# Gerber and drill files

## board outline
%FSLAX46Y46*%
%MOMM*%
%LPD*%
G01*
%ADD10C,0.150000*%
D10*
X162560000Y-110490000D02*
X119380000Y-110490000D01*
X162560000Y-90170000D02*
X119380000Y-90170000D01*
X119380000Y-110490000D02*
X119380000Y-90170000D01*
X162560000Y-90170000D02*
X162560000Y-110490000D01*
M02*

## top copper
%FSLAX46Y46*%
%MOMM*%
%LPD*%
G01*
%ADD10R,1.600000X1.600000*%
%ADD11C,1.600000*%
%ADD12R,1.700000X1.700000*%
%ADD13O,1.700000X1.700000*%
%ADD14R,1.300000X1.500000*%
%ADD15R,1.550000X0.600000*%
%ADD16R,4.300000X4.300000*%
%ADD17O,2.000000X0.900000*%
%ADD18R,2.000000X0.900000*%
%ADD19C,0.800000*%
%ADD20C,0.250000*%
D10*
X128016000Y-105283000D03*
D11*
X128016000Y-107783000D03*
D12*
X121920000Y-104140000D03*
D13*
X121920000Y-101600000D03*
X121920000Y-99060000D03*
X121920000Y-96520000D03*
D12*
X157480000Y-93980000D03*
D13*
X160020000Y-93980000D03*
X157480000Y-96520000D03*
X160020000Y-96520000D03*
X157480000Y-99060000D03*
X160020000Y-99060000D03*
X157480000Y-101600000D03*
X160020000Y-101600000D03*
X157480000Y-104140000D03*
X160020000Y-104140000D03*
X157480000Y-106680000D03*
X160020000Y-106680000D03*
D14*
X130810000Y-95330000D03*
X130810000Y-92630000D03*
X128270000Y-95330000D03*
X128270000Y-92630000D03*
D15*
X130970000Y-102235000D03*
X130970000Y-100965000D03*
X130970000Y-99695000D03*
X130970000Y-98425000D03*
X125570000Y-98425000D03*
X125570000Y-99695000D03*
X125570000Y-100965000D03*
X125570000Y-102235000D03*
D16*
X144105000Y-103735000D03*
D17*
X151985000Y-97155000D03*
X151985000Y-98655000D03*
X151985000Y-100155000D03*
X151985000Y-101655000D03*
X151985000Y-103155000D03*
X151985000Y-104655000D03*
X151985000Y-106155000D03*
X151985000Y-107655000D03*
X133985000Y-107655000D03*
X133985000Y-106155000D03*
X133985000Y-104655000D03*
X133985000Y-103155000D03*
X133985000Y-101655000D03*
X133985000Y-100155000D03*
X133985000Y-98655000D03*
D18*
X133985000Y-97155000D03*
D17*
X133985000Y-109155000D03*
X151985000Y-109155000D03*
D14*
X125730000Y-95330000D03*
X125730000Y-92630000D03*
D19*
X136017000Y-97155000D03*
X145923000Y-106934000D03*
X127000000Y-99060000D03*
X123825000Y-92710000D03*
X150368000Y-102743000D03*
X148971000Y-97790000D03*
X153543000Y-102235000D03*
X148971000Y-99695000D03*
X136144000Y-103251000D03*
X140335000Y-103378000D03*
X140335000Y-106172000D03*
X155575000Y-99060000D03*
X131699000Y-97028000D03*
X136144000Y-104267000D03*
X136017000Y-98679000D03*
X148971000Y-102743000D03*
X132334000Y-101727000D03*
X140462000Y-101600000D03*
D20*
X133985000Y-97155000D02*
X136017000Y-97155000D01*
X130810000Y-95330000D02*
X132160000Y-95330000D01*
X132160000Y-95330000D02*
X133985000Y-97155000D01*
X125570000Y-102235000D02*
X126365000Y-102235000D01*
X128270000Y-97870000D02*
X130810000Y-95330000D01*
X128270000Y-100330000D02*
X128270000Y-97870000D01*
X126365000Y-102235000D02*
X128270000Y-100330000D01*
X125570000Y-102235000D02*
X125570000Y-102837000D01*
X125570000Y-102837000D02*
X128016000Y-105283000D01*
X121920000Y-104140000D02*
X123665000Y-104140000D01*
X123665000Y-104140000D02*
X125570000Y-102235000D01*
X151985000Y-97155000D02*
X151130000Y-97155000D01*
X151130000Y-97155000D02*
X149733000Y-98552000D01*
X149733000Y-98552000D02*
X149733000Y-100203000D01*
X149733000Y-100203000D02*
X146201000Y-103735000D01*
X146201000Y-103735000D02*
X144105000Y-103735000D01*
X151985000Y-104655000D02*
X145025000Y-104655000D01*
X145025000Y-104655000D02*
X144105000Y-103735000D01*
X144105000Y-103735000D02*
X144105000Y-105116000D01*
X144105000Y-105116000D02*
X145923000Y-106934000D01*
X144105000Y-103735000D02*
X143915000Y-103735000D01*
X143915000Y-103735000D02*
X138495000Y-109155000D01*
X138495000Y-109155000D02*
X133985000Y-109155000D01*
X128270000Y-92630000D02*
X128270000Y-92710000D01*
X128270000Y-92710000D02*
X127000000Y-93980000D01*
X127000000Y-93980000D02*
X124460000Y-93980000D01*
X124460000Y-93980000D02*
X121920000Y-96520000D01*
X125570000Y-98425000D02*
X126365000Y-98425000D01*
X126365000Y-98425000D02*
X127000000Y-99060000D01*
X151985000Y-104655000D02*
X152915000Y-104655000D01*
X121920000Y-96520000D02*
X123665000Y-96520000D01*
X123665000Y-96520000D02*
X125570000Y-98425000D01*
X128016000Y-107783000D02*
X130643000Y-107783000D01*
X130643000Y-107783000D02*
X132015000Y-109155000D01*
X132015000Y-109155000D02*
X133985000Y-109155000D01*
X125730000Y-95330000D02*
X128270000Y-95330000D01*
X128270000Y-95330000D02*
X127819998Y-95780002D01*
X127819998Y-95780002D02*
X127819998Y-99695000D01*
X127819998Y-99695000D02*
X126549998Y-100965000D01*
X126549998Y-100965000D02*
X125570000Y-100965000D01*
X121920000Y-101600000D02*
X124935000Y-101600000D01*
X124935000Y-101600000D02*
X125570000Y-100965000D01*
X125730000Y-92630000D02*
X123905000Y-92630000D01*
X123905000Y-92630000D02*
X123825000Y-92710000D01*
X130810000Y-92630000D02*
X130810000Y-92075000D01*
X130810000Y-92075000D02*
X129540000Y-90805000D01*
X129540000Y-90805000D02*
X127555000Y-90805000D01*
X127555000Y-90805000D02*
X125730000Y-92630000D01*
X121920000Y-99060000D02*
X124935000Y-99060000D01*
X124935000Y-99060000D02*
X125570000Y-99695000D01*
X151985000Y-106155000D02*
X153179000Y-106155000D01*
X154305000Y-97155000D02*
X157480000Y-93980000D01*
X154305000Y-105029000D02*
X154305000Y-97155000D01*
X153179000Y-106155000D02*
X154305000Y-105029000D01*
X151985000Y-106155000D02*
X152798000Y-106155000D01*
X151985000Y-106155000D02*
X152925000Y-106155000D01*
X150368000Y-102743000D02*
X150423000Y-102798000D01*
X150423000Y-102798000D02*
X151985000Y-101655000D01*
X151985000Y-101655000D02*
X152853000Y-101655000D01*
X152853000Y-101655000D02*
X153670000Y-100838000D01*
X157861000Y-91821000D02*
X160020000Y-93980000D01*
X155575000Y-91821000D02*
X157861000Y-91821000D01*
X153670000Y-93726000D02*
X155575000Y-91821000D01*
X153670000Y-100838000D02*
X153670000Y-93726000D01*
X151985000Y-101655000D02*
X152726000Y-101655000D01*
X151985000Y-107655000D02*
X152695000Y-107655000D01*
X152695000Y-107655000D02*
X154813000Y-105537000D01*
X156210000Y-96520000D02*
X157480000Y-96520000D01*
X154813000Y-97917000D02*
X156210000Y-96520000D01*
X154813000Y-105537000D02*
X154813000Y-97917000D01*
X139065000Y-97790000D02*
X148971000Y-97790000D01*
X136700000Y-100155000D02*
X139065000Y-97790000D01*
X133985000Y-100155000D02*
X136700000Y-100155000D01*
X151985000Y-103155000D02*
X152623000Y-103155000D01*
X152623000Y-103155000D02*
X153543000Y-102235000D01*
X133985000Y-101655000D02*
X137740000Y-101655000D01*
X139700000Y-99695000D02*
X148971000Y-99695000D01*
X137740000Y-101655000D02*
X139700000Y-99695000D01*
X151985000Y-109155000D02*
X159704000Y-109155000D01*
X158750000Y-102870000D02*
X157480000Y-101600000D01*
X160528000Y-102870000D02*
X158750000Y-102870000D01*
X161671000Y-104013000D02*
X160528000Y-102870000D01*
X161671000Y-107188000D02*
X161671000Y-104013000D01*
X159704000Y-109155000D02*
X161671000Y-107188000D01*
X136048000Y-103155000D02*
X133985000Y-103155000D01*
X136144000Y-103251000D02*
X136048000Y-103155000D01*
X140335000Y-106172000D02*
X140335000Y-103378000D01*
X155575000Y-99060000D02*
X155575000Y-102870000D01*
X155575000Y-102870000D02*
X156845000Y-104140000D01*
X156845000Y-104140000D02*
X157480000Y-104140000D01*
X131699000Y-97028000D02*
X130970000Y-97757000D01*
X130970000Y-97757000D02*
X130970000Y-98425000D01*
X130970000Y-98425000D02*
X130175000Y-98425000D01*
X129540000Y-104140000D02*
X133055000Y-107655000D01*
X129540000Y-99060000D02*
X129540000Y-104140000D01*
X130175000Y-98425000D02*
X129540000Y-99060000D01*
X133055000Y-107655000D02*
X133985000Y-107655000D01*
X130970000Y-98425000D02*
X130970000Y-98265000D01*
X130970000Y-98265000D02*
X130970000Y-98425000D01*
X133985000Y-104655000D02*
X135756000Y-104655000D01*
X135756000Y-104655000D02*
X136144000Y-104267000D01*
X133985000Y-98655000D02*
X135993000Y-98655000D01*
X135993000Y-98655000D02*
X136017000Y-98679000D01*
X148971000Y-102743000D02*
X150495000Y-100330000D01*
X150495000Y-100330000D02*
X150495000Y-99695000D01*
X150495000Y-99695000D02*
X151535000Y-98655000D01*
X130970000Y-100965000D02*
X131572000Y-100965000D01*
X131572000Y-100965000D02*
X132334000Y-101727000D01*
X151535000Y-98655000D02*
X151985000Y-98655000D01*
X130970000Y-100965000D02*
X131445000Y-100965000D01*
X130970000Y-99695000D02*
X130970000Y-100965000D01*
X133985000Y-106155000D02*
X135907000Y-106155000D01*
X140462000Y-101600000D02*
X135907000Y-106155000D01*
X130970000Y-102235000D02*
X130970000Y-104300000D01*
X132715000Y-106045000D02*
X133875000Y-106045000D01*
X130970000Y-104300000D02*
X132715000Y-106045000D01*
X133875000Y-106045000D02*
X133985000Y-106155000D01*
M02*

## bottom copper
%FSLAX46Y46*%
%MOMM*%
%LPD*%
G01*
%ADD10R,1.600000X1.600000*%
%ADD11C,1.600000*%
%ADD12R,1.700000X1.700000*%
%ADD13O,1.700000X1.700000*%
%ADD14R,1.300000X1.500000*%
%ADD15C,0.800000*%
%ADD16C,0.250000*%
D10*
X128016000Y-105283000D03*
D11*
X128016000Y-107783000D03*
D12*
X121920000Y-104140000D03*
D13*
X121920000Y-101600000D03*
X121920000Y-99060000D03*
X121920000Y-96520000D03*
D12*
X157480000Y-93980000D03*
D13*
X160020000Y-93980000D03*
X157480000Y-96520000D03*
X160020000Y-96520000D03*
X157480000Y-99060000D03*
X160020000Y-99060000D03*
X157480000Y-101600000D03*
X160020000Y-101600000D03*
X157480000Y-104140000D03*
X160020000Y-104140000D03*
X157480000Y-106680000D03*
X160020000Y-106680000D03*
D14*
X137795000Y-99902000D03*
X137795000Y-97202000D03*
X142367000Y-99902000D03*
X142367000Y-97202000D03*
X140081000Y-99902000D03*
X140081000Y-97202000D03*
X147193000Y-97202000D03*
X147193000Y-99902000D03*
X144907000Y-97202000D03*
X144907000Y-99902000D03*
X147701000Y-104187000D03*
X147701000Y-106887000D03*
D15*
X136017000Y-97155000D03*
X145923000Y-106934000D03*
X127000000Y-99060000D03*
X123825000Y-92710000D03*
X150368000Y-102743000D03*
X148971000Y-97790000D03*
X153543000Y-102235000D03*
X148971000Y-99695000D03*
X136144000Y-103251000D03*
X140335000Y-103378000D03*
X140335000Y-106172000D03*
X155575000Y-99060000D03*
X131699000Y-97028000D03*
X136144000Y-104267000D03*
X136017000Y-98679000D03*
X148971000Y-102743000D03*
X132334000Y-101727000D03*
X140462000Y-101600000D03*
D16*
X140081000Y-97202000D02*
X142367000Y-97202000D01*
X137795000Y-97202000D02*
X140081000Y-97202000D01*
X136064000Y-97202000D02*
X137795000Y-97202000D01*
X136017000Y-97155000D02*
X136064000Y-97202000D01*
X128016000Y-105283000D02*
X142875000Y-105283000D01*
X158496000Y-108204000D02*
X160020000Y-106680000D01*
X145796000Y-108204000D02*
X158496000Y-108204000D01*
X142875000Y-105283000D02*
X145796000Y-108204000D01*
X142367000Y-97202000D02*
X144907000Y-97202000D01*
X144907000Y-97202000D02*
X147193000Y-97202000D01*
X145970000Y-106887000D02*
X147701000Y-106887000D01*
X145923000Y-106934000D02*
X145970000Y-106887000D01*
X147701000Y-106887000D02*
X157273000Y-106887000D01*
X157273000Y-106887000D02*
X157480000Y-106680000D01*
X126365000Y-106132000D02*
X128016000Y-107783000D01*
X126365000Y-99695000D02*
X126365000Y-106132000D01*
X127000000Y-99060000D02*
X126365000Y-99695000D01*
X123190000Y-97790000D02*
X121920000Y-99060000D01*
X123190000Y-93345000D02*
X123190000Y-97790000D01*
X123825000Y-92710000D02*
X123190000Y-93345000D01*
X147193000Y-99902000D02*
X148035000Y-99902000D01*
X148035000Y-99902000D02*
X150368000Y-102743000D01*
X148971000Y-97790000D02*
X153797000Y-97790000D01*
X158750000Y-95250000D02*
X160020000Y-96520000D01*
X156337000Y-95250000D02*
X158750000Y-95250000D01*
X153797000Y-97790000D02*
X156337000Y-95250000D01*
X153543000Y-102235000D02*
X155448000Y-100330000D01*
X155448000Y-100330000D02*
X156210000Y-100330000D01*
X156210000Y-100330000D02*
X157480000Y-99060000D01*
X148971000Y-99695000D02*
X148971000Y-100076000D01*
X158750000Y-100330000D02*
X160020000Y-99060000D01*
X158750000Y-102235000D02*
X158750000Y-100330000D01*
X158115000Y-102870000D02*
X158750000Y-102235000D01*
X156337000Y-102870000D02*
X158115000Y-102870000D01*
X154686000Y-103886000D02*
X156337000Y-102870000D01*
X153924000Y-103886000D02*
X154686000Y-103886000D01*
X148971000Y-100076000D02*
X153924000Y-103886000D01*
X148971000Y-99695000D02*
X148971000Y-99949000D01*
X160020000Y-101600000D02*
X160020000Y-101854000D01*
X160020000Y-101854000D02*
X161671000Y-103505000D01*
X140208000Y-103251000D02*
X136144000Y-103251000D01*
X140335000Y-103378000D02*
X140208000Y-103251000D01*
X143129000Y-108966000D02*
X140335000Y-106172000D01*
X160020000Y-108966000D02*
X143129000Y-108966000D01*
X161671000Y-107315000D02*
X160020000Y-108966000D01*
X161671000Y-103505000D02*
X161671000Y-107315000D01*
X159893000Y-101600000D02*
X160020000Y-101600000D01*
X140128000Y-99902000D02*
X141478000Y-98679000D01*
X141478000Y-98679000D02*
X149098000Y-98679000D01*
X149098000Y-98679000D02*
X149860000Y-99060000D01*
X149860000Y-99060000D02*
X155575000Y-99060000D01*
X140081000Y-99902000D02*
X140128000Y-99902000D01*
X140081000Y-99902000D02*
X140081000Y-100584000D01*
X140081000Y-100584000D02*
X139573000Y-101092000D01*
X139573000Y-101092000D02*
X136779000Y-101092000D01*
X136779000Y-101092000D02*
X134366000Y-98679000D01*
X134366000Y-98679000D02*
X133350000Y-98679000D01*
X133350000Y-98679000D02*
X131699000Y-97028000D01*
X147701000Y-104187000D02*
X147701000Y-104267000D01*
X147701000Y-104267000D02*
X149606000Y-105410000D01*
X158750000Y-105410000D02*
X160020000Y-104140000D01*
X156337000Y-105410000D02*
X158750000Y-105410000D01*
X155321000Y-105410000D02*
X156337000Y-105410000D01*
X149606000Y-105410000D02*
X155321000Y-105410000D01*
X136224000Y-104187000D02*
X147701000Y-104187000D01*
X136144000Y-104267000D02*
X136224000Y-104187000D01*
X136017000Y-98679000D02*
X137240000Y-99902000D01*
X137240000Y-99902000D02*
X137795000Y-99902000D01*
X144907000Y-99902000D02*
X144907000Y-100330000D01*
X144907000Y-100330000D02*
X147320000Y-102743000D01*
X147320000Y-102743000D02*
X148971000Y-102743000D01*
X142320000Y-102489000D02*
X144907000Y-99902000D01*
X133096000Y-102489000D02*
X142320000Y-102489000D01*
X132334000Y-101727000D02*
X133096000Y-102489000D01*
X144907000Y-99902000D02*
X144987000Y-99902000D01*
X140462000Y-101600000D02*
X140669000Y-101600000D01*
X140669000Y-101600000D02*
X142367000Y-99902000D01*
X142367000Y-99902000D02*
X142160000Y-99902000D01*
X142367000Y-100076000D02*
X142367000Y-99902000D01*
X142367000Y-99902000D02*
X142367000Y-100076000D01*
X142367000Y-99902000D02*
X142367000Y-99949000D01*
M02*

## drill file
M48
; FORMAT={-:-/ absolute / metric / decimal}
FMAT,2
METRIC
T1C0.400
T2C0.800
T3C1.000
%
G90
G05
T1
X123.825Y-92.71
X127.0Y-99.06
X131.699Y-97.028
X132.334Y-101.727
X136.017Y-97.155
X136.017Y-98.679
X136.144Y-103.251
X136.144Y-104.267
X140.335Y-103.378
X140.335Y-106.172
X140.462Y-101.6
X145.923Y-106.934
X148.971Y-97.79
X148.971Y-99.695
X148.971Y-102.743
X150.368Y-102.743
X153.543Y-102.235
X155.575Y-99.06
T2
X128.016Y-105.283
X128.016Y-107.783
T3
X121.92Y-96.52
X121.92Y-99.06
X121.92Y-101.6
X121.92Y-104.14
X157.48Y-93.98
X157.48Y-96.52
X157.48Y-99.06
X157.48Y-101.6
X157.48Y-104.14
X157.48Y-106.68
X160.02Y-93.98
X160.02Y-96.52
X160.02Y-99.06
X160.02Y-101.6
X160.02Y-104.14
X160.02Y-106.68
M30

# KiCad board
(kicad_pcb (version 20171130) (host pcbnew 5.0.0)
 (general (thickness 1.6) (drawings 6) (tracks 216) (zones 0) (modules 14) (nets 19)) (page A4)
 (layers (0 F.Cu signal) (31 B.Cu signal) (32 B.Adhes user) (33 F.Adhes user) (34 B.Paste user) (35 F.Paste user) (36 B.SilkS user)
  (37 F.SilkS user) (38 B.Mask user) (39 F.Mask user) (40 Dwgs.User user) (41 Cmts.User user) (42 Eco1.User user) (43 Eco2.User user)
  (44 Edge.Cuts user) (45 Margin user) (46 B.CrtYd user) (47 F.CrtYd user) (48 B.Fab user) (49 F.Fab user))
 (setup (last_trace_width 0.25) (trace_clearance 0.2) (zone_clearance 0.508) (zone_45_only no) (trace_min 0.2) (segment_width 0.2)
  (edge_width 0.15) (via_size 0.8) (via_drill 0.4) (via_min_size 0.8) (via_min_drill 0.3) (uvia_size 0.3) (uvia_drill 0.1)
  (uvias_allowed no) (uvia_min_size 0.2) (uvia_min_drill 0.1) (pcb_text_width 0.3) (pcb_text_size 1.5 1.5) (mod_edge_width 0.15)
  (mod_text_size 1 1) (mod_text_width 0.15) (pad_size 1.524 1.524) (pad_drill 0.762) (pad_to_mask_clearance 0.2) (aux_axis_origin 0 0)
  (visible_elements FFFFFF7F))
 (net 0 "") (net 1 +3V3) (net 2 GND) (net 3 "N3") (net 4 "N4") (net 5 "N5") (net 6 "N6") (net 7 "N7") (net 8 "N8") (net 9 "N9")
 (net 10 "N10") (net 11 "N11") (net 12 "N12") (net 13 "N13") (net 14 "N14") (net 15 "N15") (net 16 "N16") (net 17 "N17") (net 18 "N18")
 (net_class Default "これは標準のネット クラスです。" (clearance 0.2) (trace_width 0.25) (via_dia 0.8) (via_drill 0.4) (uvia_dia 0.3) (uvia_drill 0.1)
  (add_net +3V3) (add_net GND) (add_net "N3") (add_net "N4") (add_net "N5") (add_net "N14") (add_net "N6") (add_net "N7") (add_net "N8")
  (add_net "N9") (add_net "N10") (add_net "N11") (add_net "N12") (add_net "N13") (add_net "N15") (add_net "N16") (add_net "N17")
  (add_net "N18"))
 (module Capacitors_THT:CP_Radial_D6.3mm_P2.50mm (layer F.Cu) (at 128.016 105.283 270)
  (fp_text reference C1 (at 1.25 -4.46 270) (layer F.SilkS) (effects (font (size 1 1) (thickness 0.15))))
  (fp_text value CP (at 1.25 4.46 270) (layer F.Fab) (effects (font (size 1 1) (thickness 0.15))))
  (pad 1 thru_hole rect (at 0 0 270) (size 1.6 1.6) (drill 0.8) (layers *.Cu *.Mask) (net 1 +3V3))
  (pad 2 thru_hole circle (at 2.5 0 270) (size 1.6 1.6) (drill 0.8) (layers *.Cu *.Mask) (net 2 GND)))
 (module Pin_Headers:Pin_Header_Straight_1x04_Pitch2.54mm (layer F.Cu) (at 121.92 104.14 180)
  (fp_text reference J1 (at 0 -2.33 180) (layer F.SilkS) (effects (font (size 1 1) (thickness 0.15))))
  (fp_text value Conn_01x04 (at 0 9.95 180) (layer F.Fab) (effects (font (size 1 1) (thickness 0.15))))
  (pad 1 thru_hole rect (at 0 0 180) (size 1.7 1.7) (drill 1) (layers *.Cu *.Mask) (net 1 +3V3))
  (pad 2 thru_hole oval (at 0 2.54 180) (size 1.7 1.7) (drill 1) (layers *.Cu *.Mask) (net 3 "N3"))
  (pad 3 thru_hole oval (at 0 5.08 180) (size 1.7 1.7) (drill 1) (layers *.Cu *.Mask) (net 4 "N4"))
  (pad 4 thru_hole oval (at 0 7.62 180) (size 1.7 1.7) (drill 1) (layers *.Cu *.Mask) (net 2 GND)))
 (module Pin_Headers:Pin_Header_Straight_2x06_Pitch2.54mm (layer F.Cu) (at 157.48 93.98)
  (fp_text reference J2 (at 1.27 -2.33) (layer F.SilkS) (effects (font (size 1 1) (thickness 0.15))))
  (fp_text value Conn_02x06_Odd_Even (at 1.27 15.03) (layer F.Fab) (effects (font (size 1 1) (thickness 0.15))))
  (pad 1 thru_hole rect (at 0 0) (size 1.7 1.7) (drill 1) (layers *.Cu *.Mask) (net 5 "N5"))
  (pad 2 thru_hole oval (at 2.54 0) (size 1.7 1.7) (drill 1) (layers *.Cu *.Mask) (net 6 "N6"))
  (pad 3 thru_hole oval (at 0 2.54) (size 1.7 1.7) (drill 1) (layers *.Cu *.Mask) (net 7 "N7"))
  (pad 4 thru_hole oval (at 2.54 2.54) (size 1.7 1.7) (drill 1) (layers *.Cu *.Mask) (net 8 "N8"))
  (pad 5 thru_hole oval (at 0 5.08) (size 1.7 1.7) (drill 1) (layers *.Cu *.Mask) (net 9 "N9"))
  (pad 6 thru_hole oval (at 2.54 5.08) (size 1.7 1.7) (drill 1) (layers *.Cu *.Mask) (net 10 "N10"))
  (pad 7 thru_hole oval (at 0 7.62) (size 1.7 1.7) (drill 1) (layers *.Cu *.Mask) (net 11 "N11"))
  (pad 8 thru_hole oval (at 2.54 7.62) (size 1.7 1.7) (drill 1) (layers *.Cu *.Mask) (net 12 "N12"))
  (pad 9 thru_hole oval (at 0 10.16) (size 1.7 1.7) (drill 1) (layers *.Cu *.Mask) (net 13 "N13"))
  (pad 10 thru_hole oval (at 2.54 10.16) (size 1.7 1.7) (drill 1) (layers *.Cu *.Mask) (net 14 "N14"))
  (pad 11 thru_hole oval (at 0 12.7) (size 1.7 1.7) (drill 1) (layers *.Cu *.Mask) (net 2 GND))
  (pad 12 thru_hole oval (at 2.54 12.7) (size 1.7 1.7) (drill 1) (layers *.Cu *.Mask) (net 1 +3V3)))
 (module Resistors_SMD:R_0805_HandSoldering (layer B.Cu) (at 137.795 98.552 90)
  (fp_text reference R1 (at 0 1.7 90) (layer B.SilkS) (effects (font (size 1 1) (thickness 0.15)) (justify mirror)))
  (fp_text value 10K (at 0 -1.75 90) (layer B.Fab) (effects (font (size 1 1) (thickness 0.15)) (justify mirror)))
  (pad 1 smd rect (at -1.35 0 90) (size 1.5 1.3) (layers B.Cu B.Paste B.Mask) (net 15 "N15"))
  (pad 2 smd rect (at 1.35 0 90) (size 1.5 1.3) (layers B.Cu B.Paste B.Mask) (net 1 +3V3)))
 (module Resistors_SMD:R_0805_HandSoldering (layer B.Cu) (at 142.367 98.552 90)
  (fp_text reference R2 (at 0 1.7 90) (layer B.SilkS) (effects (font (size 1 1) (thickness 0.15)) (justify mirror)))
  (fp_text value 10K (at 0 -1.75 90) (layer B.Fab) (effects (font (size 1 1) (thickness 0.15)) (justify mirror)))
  (pad 1 smd rect (at -1.35 0 90) (size 1.5 1.3) (layers B.Cu B.Paste B.Mask) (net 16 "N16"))
  (pad 2 smd rect (at 1.35 0 90) (size 1.5 1.3) (layers B.Cu B.Paste B.Mask) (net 1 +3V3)))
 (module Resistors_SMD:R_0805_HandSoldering (layer B.Cu) (at 140.081 98.552 90)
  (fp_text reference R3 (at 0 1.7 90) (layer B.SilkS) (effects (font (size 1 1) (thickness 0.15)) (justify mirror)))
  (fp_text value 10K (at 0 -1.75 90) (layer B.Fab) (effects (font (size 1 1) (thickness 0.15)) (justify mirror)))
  (pad 1 smd rect (at -1.35 0 90) (size 1.5 1.3) (layers B.Cu B.Paste B.Mask) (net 13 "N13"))
  (pad 2 smd rect (at 1.35 0 90) (size 1.5 1.3) (layers B.Cu B.Paste B.Mask) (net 1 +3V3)))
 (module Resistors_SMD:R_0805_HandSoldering (layer F.Cu) (at 130.81 93.98 90)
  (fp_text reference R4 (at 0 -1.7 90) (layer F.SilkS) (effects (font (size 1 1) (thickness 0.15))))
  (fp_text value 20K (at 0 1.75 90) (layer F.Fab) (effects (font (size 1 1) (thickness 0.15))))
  (pad 1 smd rect (at -1.35 0 90) (size 1.5 1.3) (layers F.Cu F.Paste F.Mask) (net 1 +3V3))
  (pad 2 smd rect (at 1.35 0 90) (size 1.5 1.3) (layers F.Cu F.Paste F.Mask) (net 4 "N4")))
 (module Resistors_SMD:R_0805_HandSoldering (layer F.Cu) (at 128.27 93.98 90)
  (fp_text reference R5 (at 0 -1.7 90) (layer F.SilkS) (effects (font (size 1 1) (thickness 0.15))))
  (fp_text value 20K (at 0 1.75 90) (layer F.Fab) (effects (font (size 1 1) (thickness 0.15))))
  (pad 1 smd rect (at -1.35 0 90) (size 1.5 1.3) (layers F.Cu F.Paste F.Mask) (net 3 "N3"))
  (pad 2 smd rect (at 1.35 0 90) (size 1.5 1.3) (layers F.Cu F.Paste F.Mask) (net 2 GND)))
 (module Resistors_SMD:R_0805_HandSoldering (layer B.Cu) (at 147.193 98.552 270)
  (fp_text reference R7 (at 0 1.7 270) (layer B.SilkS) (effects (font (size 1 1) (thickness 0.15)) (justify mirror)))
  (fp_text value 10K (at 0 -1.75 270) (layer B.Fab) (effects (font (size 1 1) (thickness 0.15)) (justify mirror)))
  (pad 1 smd rect (at -1.35 0 270) (size 1.5 1.3) (layers B.Cu B.Paste B.Mask) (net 1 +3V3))
  (pad 2 smd rect (at 1.35 0 270) (size 1.5 1.3) (layers B.Cu B.Paste B.Mask) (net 6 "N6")))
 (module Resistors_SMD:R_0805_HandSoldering (layer B.Cu) (at 144.907 98.552 270)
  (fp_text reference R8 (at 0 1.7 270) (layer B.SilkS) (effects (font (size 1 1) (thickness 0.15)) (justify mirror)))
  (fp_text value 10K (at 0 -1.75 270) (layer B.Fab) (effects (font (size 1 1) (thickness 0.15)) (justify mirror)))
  (pad 1 smd rect (at -1.35 0 270) (size 1.5 1.3) (layers B.Cu B.Paste B.Mask) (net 1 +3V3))
  (pad 2 smd rect (at 1.35 0 270) (size 1.5 1.3) (layers B.Cu B.Paste B.Mask) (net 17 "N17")))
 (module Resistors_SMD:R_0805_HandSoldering (layer B.Cu) (at 147.701 105.537 270)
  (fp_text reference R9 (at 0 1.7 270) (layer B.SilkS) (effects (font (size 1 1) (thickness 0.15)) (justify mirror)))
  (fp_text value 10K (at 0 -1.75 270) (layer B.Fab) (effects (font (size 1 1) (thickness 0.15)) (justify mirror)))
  (pad 1 smd rect (at -1.35 0 270) (size 1.5 1.3) (layers B.Cu B.Paste B.Mask) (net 14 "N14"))
  (pad 2 smd rect (at 1.35 0 270) (size 1.5 1.3) (layers B.Cu B.Paste B.Mask) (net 2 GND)))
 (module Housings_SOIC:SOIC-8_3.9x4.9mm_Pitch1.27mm (layer F.Cu) (at 128.27 100.33 180)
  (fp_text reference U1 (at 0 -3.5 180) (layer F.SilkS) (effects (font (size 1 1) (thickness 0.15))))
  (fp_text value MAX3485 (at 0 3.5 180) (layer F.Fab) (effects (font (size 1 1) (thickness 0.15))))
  (pad 1 smd rect (at -2.7 -1.905 180) (size 1.55 0.6) (layers F.Cu F.Paste F.Mask) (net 16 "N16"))
  (pad 2 smd rect (at -2.7 -0.635 180) (size 1.55 0.6) (layers F.Cu F.Paste F.Mask) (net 17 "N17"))
  (pad 3 smd rect (at -2.7 0.635 180) (size 1.55 0.6) (layers F.Cu F.Paste F.Mask) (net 17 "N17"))
  (pad 4 smd rect (at -2.7 1.905 180) (size 1.55 0.6) (layers F.Cu F.Paste F.Mask) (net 13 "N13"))
  (pad 5 smd rect (at 2.7 1.905 180) (size 1.55 0.6) (layers F.Cu F.Paste F.Mask) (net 2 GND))
  (pad 6 smd rect (at 2.7 0.635 180) (size 1.55 0.6) (layers F.Cu F.Paste F.Mask) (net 4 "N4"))
  (pad 7 smd rect (at 2.7 -0.635 180) (size 1.55 0.6) (layers F.Cu F.Paste F.Mask) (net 3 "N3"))
  (pad 8 smd rect (at 2.7 -1.905 180) (size 1.55 0.6) (layers F.Cu F.Paste F.Mask) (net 1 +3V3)))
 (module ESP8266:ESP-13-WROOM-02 (layer F.Cu) (at 133.985 97.155)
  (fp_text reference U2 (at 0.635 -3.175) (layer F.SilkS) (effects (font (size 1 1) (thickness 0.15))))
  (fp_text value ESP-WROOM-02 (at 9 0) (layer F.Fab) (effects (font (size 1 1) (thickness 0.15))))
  (pad PAD smd rect (at 10.12 6.58) (size 4.3 4.3) (layers F.Cu F.Paste F.Mask) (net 2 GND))
  (pad 18 smd oval (at 18 0) (size 2 0.9) (layers F.Cu F.Paste F.Mask) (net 2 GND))
  (pad 17 smd oval (at 18 1.5) (size 2 0.9) (layers F.Cu F.Paste F.Mask) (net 17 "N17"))
  (pad 16 smd oval (at 18 3) (size 2 0.9) (layers F.Cu F.Paste F.Mask) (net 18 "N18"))
  (pad 15 smd oval (at 18 4.5) (size 2 0.9) (layers F.Cu F.Paste F.Mask) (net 6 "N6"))
  (pad 14 smd oval (at 18 6) (size 2 0.9) (layers F.Cu F.Paste F.Mask) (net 9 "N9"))
  (pad 13 smd oval (at 18 7.5) (size 2 0.9) (layers F.Cu F.Paste F.Mask) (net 2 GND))
  (pad 12 smd oval (at 18 9) (size 2 0.9) (layers F.Cu F.Paste F.Mask) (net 5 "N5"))
  (pad 11 smd oval (at 18 10.5) (size 2 0.9) (layers F.Cu F.Paste F.Mask) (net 7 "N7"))
  (pad 8 smd oval (at 0 10.5) (size 2 0.9) (layers F.Cu F.Paste F.Mask) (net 13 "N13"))
  (pad 7 smd oval (at 0 9) (size 2 0.9) (layers F.Cu F.Paste F.Mask) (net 16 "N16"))
  (pad 6 smd oval (at 0 7.5) (size 2 0.9) (layers F.Cu F.Paste F.Mask) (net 14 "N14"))
  (pad 5 smd oval (at 0 6) (size 2 0.9) (layers F.Cu F.Paste F.Mask) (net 12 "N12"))
  (pad 4 smd oval (at 0 4.5) (size 2 0.9) (layers F.Cu F.Paste F.Mask) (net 10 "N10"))
  (pad 3 smd oval (at 0 3) (size 2 0.9) (layers F.Cu F.Paste F.Mask) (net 8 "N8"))
  (pad 2 smd oval (at 0 1.5) (size 2 0.9) (layers F.Cu F.Paste F.Mask) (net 15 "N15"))
  (pad 1 smd rect (at 0 0) (size 2 0.9) (layers F.Cu F.Paste F.Mask) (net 1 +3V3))
  (pad 9 smd oval (at 0 12) (size 2 0.9) (layers F.Cu F.Paste F.Mask) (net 2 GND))
  (pad 10 smd oval (at 18 12) (size 2 0.9) (layers F.Cu F.Paste F.Mask) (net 11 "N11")))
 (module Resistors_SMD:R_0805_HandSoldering (layer F.Cu) (at 125.73 93.98 90)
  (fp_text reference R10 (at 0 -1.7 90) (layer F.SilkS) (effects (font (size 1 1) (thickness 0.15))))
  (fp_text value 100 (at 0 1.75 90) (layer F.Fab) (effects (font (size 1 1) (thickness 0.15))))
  (pad 1 smd rect (at -1.35 0 90) (size 1.5 1.3) (layers F.Cu F.Paste F.Mask) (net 3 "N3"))
  (pad 2 smd rect (at 1.35 0 90) (size 1.5 1.3) (layers F.Cu F.Paste F.Mask) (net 4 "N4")))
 (gr_line (start 162.56 110.49) (end 119.38 110.49) (angle 90) (layer Edge.Cuts) (width 0.15))
 (gr_line (start 162.56 90.17) (end 119.38 90.17) (angle 90) (layer Edge.Cuts) (width 0.15))
 (gr_line (start 119.38 110.49) (end 119.38 90.17) (angle 90) (layer Edge.Cuts) (width 0.15))
 (gr_line (start 162.56 90.17) (end 162.56 110.49) (angle 90) (layer Edge.Cuts) (width 0.15))
 (segment (start 140.081 97.202) (end 142.367 97.202) (width 0.25) (layer B.Cu) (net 1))
 (segment (start 137.795 97.202) (end 140.081 97.202) (width 0.25) (layer B.Cu) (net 1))
 (segment (start 133.985 97.155) (end 136.017 97.155) (width 0.25) (layer F.Cu) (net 1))
 (segment (start 136.064 97.202) (end 137.795 97.202) (width 0.25) (layer B.Cu) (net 1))
 (segment (start 136.017 97.155) (end 136.064 97.202) (width 0.25) (layer B.Cu) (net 1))
 (via (at 136.017 97.155) (size 0.8) (drill 0.4) (layers F.Cu B.Cu) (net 1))
 (segment (start 128.016 105.283) (end 142.875 105.283) (width 0.25) (layer B.Cu) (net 1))
 (segment (start 158.496 108.204) (end 160.02 106.68) (width 0.25) (layer B.Cu) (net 1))
 (segment (start 145.796 108.204) (end 158.496 108.204) (width 0.25) (layer B.Cu) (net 1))
 (segment (start 142.875 105.283) (end 145.796 108.204) (width 0.25) (layer B.Cu) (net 1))
 (segment (start 142.367 97.202) (end 144.907 97.202) (width 0.25) (layer B.Cu) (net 1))
 (segment (start 144.907 97.202) (end 147.193 97.202) (width 0.25) (layer B.Cu) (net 1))
 (segment (start 130.81 95.33) (end 132.16 95.33) (width 0.25) (layer F.Cu) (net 1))
 (segment (start 132.16 95.33) (end 133.985 97.155) (width 0.25) (layer F.Cu) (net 1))
 (segment (start 125.57 102.235) (end 126.365 102.235) (width 0.25) (layer F.Cu) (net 1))
 (segment (start 128.27 97.87) (end 130.81 95.33) (width 0.25) (layer F.Cu) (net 1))
 (segment (start 128.27 100.33) (end 128.27 97.87) (width 0.25) (layer F.Cu) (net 1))
 (segment (start 126.365 102.235) (end 128.27 100.33) (width 0.25) (layer F.Cu) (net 1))
 (segment (start 125.57 102.235) (end 125.57 102.837) (width 0.25) (layer F.Cu) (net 1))
 (segment (start 125.57 102.837) (end 128.016 105.283) (width 0.25) (layer F.Cu) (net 1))
 (segment (start 121.92 104.14) (end 123.665 104.14) (width 0.25) (layer F.Cu) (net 1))
 (segment (start 123.665 104.14) (end 125.57 102.235) (width 0.25) (layer F.Cu) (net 1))
 (segment (start 151.985 97.155) (end 151.13 97.155) (width 0.25) (layer F.Cu) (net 2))
 (segment (start 151.13 97.155) (end 149.733 98.552) (width 0.25) (layer F.Cu) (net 2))
 (segment (start 149.733 98.552) (end 149.733 100.203) (width 0.25) (layer F.Cu) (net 2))
 (segment (start 149.733 100.203) (end 146.201 103.735) (width 0.25) (layer F.Cu) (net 2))
 (segment (start 146.201 103.735) (end 144.105 103.735) (width 0.25) (layer F.Cu) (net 2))
 (segment (start 151.985 104.655) (end 145.025 104.655) (width 0.25) (layer F.Cu) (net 2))
 (segment (start 145.025 104.655) (end 144.105 103.735) (width 0.25) (layer F.Cu) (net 2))
 (segment (start 144.105 103.735) (end 144.105 105.116) (width 0.25) (layer F.Cu) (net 2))
 (segment (start 144.105 105.116) (end 145.923 106.934) (width 0.25) (layer F.Cu) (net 2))
 (segment (start 145.97 106.887) (end 147.701 106.887) (width 0.25) (layer B.Cu) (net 2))
 (segment (start 145.923 106.934) (end 145.97 106.887) (width 0.25) (layer B.Cu) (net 2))
 (via (at 145.923 106.934) (size 0.8) (drill 0.4) (layers F.Cu B.Cu) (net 2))
 (segment (start 147.701 106.887) (end 157.273 106.887) (width 0.25) (layer B.Cu) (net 2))
 (segment (start 157.273 106.887) (end 157.48 106.68) (width 0.25) (layer B.Cu) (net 2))
 (segment (start 144.105 103.735) (end 143.915 103.735) (width 0.25) (layer F.Cu) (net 2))
 (segment (start 143.915 103.735) (end 138.495 109.155) (width 0.25) (layer F.Cu) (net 2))
 (segment (start 138.495 109.155) (end 133.985 109.155) (width 0.25) (layer F.Cu) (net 2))
 (segment (start 128.27 92.63) (end 128.27 92.71) (width 0.25) (layer F.Cu) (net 2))
 (segment (start 128.27 92.71) (end 127 93.98) (width 0.25) (layer F.Cu) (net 2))
 (segment (start 127 93.98) (end 124.46 93.98) (width 0.25) (layer F.Cu) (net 2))
 (segment (start 124.46 93.98) (end 121.92 96.52) (width 0.25) (layer F.Cu) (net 2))
 (segment (start 125.57 98.425) (end 126.365 98.425) (width 0.25) (layer F.Cu) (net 2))
 (segment (start 126.365 106.132) (end 128.016 107.783) (width 0.25) (layer B.Cu) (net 2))
 (segment (start 126.365 99.695) (end 126.365 106.132) (width 0.25) (layer B.Cu) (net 2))
 (segment (start 127 99.06) (end 126.365 99.695) (width 0.25) (layer B.Cu) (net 2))
 (via (at 127 99.06) (size 0.8) (drill 0.4) (layers F.Cu B.Cu) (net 2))
 (segment (start 126.365 98.425) (end 127 99.06) (width 0.25) (layer F.Cu) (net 2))
 (segment (start 151.985 104.655) (end 152.915 104.655) (width 0.25) (layer F.Cu) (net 2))
 (segment (start 121.92 96.52) (end 123.665 96.52) (width 0.25) (layer F.Cu) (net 2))
 (segment (start 123.665 96.52) (end 125.57 98.425) (width 0.25) (layer F.Cu) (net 2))
 (segment (start 128.016 107.783) (end 130.643 107.783) (width 0.25) (layer F.Cu) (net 2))
 (segment (start 130.643 107.783) (end 132.015 109.155) (width 0.25) (layer F.Cu) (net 2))
 (segment (start 132.015 109.155) (end 133.985 109.155) (width 0.25) (layer F.Cu) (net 2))
 (segment (start 125.73 95.33) (end 128.27 95.33) (width 0.25) (layer F.Cu) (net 3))
 (segment (start 128.27 95.33) (end 127.819998 95.780002) (width 0.25) (layer F.Cu) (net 3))
 (segment (start 127.819998 95.780002) (end 127.819998 99.695) (width 0.25) (layer F.Cu) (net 3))
 (segment (start 127.819998 99.695) (end 126.549998 100.965) (width 0.25) (layer F.Cu) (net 3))
 (segment (start 126.549998 100.965) (end 125.57 100.965) (width 0.25) (layer F.Cu) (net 3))
 (segment (start 121.92 101.6) (end 124.935 101.6) (width 0.25) (layer F.Cu) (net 3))
 (segment (start 124.935 101.6) (end 125.57 100.965) (width 0.25) (layer F.Cu) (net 3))
 (segment (start 125.73 92.63) (end 123.905 92.63) (width 0.25) (layer F.Cu) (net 4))
 (segment (start 123.19 97.79) (end 121.92 99.06) (width 0.25) (layer B.Cu) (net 4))
 (segment (start 123.19 93.345) (end 123.19 97.79) (width 0.25) (layer B.Cu) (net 4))
 (segment (start 123.825 92.71) (end 123.19 93.345) (width 0.25) (layer B.Cu) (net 4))
 (via (at 123.825 92.71) (size 0.8) (drill 0.4) (layers F.Cu B.Cu) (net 4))
 (segment (start 123.905 92.63) (end 123.825 92.71) (width 0.25) (layer F.Cu) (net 4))
 (segment (start 130.81 92.63) (end 130.81 92.075) (width 0.25) (layer F.Cu) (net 4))
 (segment (start 130.81 92.075) (end 129.54 90.805) (width 0.25) (layer F.Cu) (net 4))
 (segment (start 129.54 90.805) (end 127.555 90.805) (width 0.25) (layer F.Cu) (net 4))
 (segment (start 127.555 90.805) (end 125.73 92.63) (width 0.25) (layer F.Cu) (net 4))
 (segment (start 121.92 99.06) (end 124.935 99.06) (width 0.25) (layer F.Cu) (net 4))
 (segment (start 124.935 99.06) (end 125.57 99.695) (width 0.25) (layer F.Cu) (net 4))
 (segment (start 151.985 106.155) (end 153.179 106.155) (width 0.25) (layer F.Cu) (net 5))
 (segment (start 154.305 97.155) (end 157.48 93.98) (width 0.25) (layer F.Cu) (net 5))
 (segment (start 154.305 105.029) (end 154.305 97.155) (width 0.25) (layer F.Cu) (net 5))
 (segment (start 153.179 106.155) (end 154.305 105.029) (width 0.25) (layer F.Cu) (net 5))
 (segment (start 151.985 106.155) (end 152.798 106.155) (width 0.25) (layer F.Cu) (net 5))
 (segment (start 151.985 106.155) (end 152.925 106.155) (width 0.25) (layer F.Cu) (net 5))
 (segment (start 147.193 99.902) (end 148.035 99.902) (width 0.25) (layer B.Cu) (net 6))
 (via (at 150.368 102.743) (size 0.8) (drill 0.4) (layers F.Cu B.Cu) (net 6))
 (segment (start 150.368 102.743) (end 150.423 102.798) (width 0.25) (layer F.Cu) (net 6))
 (segment (start 150.423 102.798) (end 151.985 101.655) (width 0.25) (layer F.Cu) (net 6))
 (segment (start 148.035 99.902) (end 150.368 102.743) (width 0.25) (layer B.Cu) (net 6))
 (segment (start 151.985 101.655) (end 152.853 101.655) (width 0.25) (layer F.Cu) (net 6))
 (segment (start 152.853 101.655) (end 153.67 100.838) (width 0.25) (layer F.Cu) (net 6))
 (segment (start 157.861 91.821) (end 160.02 93.98) (width 0.25) (layer F.Cu) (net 6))
 (segment (start 155.575 91.821) (end 157.861 91.821) (width 0.25) (layer F.Cu) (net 6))
 (segment (start 153.67 93.726) (end 155.575 91.821) (width 0.25) (layer F.Cu) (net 6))
 (segment (start 153.67 100.838) (end 153.67 93.726) (width 0.25) (layer F.Cu) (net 6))
 (segment (start 151.985 101.655) (end 152.726 101.655) (width 0.25) (layer F.Cu) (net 6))
 (segment (start 151.985 107.655) (end 152.695 107.655) (width 0.25) (layer F.Cu) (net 7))
 (segment (start 152.695 107.655) (end 154.813 105.537) (width 0.25) (layer F.Cu) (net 7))
 (segment (start 156.21 96.52) (end 157.48 96.52) (width 0.25) (layer F.Cu) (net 7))
 (segment (start 154.813 97.917) (end 156.21 96.52) (width 0.25) (layer F.Cu) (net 7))
 (segment (start 154.813 105.537) (end 154.813 97.917) (width 0.25) (layer F.Cu) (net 7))
 (segment (start 148.971 97.79) (end 153.797 97.79) (width 0.25) (layer B.Cu) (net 8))
 (via (at 148.971 97.79) (size 0.8) (drill 0.4) (layers F.Cu B.Cu) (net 8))
 (segment (start 139.065 97.79) (end 148.971 97.79) (width 0.25) (layer F.Cu) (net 8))
 (segment (start 136.7 100.155) (end 139.065 97.79) (width 0.25) (layer F.Cu) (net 8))
 (segment (start 133.985 100.155) (end 136.7 100.155) (width 0.25) (layer F.Cu) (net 8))
 (segment (start 158.75 95.25) (end 160.02 96.52) (width 0.25) (layer B.Cu) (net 8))
 (segment (start 156.337 95.25) (end 158.75 95.25) (width 0.25) (layer B.Cu) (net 8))
 (segment (start 153.797 97.79) (end 156.337 95.25) (width 0.25) (layer B.Cu) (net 8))
 (segment (start 151.985 103.155) (end 152.623 103.155) (width 0.25) (layer F.Cu) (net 9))
 (segment (start 152.623 103.155) (end 153.543 102.235) (width 0.25) (layer F.Cu) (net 9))
 (via (at 153.543 102.235) (size 0.8) (drill 0.4) (layers F.Cu B.Cu) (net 9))
 (segment (start 153.543 102.235) (end 155.448 100.33) (width 0.25) (layer B.Cu) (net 9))
 (segment (start 155.448 100.33) (end 156.21 100.33) (width 0.25) (layer B.Cu) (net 9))
 (segment (start 156.21 100.33) (end 157.48 99.06) (width 0.25) (layer B.Cu) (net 9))
 (segment (start 148.971 99.695) (end 148.971 100.076) (width 0.25) (layer B.Cu) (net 10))
 (segment (start 158.75 100.33) (end 160.02 99.06) (width 0.25) (layer B.Cu) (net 10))
 (segment (start 158.75 102.235) (end 158.75 100.33) (width 0.25) (layer B.Cu) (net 10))
 (segment (start 158.115 102.87) (end 158.75 102.235) (width 0.25) (layer B.Cu) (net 10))
 (segment (start 156.337 102.87) (end 158.115 102.87) (width 0.25) (layer B.Cu) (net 10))
 (segment (start 154.686 103.886) (end 156.337 102.87) (width 0.25) (layer B.Cu) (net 10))
 (segment (start 153.924 103.886) (end 154.686 103.886) (width 0.25) (layer B.Cu) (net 10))
 (segment (start 148.971 100.076) (end 153.924 103.886) (width 0.25) (layer B.Cu) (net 10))
 (segment (start 133.985 101.655) (end 137.74 101.655) (width 0.25) (layer F.Cu) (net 10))
 (via (at 148.971 99.695) (size 0.8) (drill 0.4) (layers F.Cu B.Cu) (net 10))
 (segment (start 139.7 99.695) (end 148.971 99.695) (width 0.25) (layer F.Cu) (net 10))
 (segment (start 137.74 101.655) (end 139.7 99.695) (width 0.25) (layer F.Cu) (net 10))
 (segment (start 148.971 99.695) (end 148.971 99.949) (width 0.25) (layer B.Cu) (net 10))
 (segment (start 151.985 109.155) (end 159.704 109.155) (width 0.25) (layer F.Cu) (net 11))
 (segment (start 158.75 102.87) (end 157.48 101.6) (width 0.25) (layer F.Cu) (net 11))
 (segment (start 160.528 102.87) (end 158.75 102.87) (width 0.25) (layer F.Cu) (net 11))
 (segment (start 161.671 104.013) (end 160.528 102.87) (width 0.25) (layer F.Cu) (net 11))
 (segment (start 161.671 107.188) (end 161.671 104.013) (width 0.25) (layer F.Cu) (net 11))
 (segment (start 159.704 109.155) (end 161.671 107.188) (width 0.25) (layer F.Cu) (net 11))
 (segment (start 160.02 101.6) (end 160.02 101.854) (width 0.25) (layer B.Cu) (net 12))
 (segment (start 160.02 101.854) (end 161.671 103.505) (width 0.25) (layer B.Cu) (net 12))
 (segment (start 136.048 103.155) (end 133.985 103.155) (width 0.25) (layer F.Cu) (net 12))
 (segment (start 136.144 103.251) (end 136.048 103.155) (width 0.25) (layer F.Cu) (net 12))
 (via (at 136.144 103.251) (size 0.8) (drill 0.4) (layers F.Cu B.Cu) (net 12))
 (segment (start 140.208 103.251) (end 136.144 103.251) (width 0.25) (layer B.Cu) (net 12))
 (segment (start 140.335 103.378) (end 140.208 103.251) (width 0.25) (layer B.Cu) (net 12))
 (via (at 140.335 103.378) (size 0.8) (drill 0.4) (layers F.Cu B.Cu) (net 12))
 (segment (start 140.335 106.172) (end 140.335 103.378) (width 0.25) (layer F.Cu) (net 12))
 (via (at 140.335 106.172) (size 0.8) (drill 0.4) (layers F.Cu B.Cu) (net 12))
 (segment (start 143.129 108.966) (end 140.335 106.172) (width 0.25) (layer B.Cu) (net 12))
 (segment (start 160.02 108.966) (end 143.129 108.966) (width 0.25) (layer B.Cu) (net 12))
 (segment (start 161.671 107.315) (end 160.02 108.966) (width 0.25) (layer B.Cu) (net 12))
 (segment (start 161.671 103.505) (end 161.671 107.315) (width 0.25) (layer B.Cu) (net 12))
 (segment (start 159.893 101.6) (end 160.02 101.6) (width 0.25) (layer B.Cu) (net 12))
 (segment (start 140.128 99.902) (end 141.478 98.679) (width 0.25) (layer B.Cu) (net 13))
 (segment (start 141.478 98.679) (end 149.098 98.679) (width 0.25) (layer B.Cu) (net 13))
 (segment (start 149.098 98.679) (end 149.86 99.06) (width 0.25) (layer B.Cu) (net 13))
 (segment (start 149.86 99.06) (end 155.575 99.06) (width 0.25) (layer B.Cu) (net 13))
 (via (at 155.575 99.06) (size 0.8) (drill 0.4) (layers F.Cu B.Cu) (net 13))
 (segment (start 155.575 99.06) (end 155.575 102.87) (width 0.25) (layer F.Cu) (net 13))
 (segment (start 155.575 102.87) (end 156.845 104.14) (width 0.25) (layer F.Cu) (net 13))
 (segment (start 140.081 99.902) (end 140.128 99.902) (width 0.25) (layer B.Cu) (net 13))
 (segment (start 156.845 104.14) (end 157.48 104.14) (width 0.25) (layer F.Cu) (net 13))
 (segment (start 140.081 99.902) (end 140.081 100.584) (width 0.25) (layer B.Cu) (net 13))
 (segment (start 140.081 100.584) (end 139.573 101.092) (width 0.25) (layer B.Cu) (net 13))
 (segment (start 139.573 101.092) (end 136.779 101.092) (width 0.25) (layer B.Cu) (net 13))
 (segment (start 136.779 101.092) (end 134.366 98.679) (width 0.25) (layer B.Cu) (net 13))
 (segment (start 134.366 98.679) (end 133.35 98.679) (width 0.25) (layer B.Cu) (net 13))
 (segment (start 133.35 98.679) (end 131.699 97.028) (width 0.25) (layer B.Cu) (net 13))
 (via (at 131.699 97.028) (size 0.8) (drill 0.4) (layers F.Cu B.Cu) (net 13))
 (segment (start 131.699 97.028) (end 130.97 97.757) (width 0.25) (layer F.Cu) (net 13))
 (segment (start 130.97 97.757) (end 130.97 98.425) (width 0.25) (layer F.Cu) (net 13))
 (segment (start 130.97 98.425) (end 130.175 98.425) (width 0.25) (layer F.Cu) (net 13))
 (segment (start 129.54 104.14) (end 133.055 107.655) (width 0.25) (layer F.Cu) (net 13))
 (segment (start 129.54 99.06) (end 129.54 104.14) (width 0.25) (layer F.Cu) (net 13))
 (segment (start 130.175 98.425) (end 129.54 99.06) (width 0.25) (layer F.Cu) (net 13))
 (segment (start 133.055 107.655) (end 133.985 107.655) (width 0.25) (layer F.Cu) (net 13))
 (segment (start 130.97 98.425) (end 130.97 98.265) (width 0.25) (layer F.Cu) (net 13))
 (segment (start 130.97 98.265) (end 130.97 98.425) (width 0.25) (layer F.Cu) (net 13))
 (segment (start 147.701 104.187) (end 147.701 104.267) (width 0.25) (layer B.Cu) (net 14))
 (segment (start 147.701 104.267) (end 149.606 105.41) (width 0.25) (layer B.Cu) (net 14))
 (segment (start 158.75 105.41) (end 160.02 104.14) (width 0.25) (layer B.Cu) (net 14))
 (segment (start 156.337 105.41) (end 158.75 105.41) (width 0.25) (layer B.Cu) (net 14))
 (segment (start 155.321 105.41) (end 156.337 105.41) (width 0.25) (layer B.Cu) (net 14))
 (segment (start 149.606 105.41) (end 155.321 105.41) (width 0.25) (layer B.Cu) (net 14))
 (segment (start 133.985 104.655) (end 135.756 104.655) (width 0.25) (layer F.Cu) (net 14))
 (segment (start 136.224 104.187) (end 147.701 104.187) (width 0.25) (layer B.Cu) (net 14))
 (segment (start 136.144 104.267) (end 136.224 104.187) (width 0.25) (layer B.Cu) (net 14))
 (via (at 136.144 104.267) (size 0.8) (drill 0.4) (layers F.Cu B.Cu) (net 14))
 (segment (start 135.756 104.655) (end 136.144 104.267) (width 0.25) (layer F.Cu) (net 14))
 (segment (start 133.985 98.655) (end 135.993 98.655) (width 0.25) (layer F.Cu) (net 15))
 (segment (start 136.017 98.679) (end 137.24 99.902) (width 0.25) (layer B.Cu) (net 15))
 (via (at 136.017 98.679) (size 0.8) (drill 0.4) (layers F.Cu B.Cu) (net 15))
 (segment (start 135.993 98.655) (end 136.017 98.679) (width 0.25) (layer F.Cu) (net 15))
 (segment (start 137.24 99.902) (end 137.795 99.902) (width 0.25) (layer B.Cu) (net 15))
 (segment (start 144.907 99.902) (end 144.907 100.33) (width 0.25) (layer B.Cu) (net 17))
 (segment (start 144.907 100.33) (end 147.32 102.743) (width 0.25) (layer B.Cu) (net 17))
 (via (at 148.971 102.743) (size 0.8) (drill 0.4) (layers F.Cu B.Cu) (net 17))
 (segment (start 148.971 102.743) (end 150.495 100.33) (width 0.25) (layer F.Cu) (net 17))
 (segment (start 150.495 100.33) (end 150.495 99.695) (width 0.25) (layer F.Cu) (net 17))
 (segment (start 150.495 99.695) (end 151.535 98.655) (width 0.25) (layer F.Cu) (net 17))
 (segment (start 147.32 102.743) (end 148.971 102.743) (width 0.25) (layer B.Cu) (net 17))
 (segment (start 130.97 100.965) (end 131.572 100.965) (width 0.25) (layer F.Cu) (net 17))
 (segment (start 131.572 100.965) (end 132.334 101.727) (width 0.25) (layer F.Cu) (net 17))
 (segment (start 142.32 102.489) (end 144.907 99.902) (width 0.25) (layer B.Cu) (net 17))
 (segment (start 133.096 102.489) (end 142.32 102.489) (width 0.25) (layer B.Cu) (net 17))
 (segment (start 132.334 101.727) (end 133.096 102.489) (width 0.25) (layer B.Cu) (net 17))
 (via (at 132.334 101.727) (size 0.8) (drill 0.4) (layers F.Cu B.Cu) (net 17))
 (segment (start 144.907 99.902) (end 144.987 99.902) (width 0.25) (layer B.Cu) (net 17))
 (segment (start 151.535 98.655) (end 151.985 98.655) (width 0.25) (layer F.Cu) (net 17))
 (segment (start 130.97 100.965) (end 131.445 100.965) (width 0.25) (layer F.Cu) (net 17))
 (segment (start 130.97 99.695) (end 130.97 100.965) (width 0.25) (layer F.Cu) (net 17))
 (segment (start 140.462 101.6) (end 140.669 101.6) (width 0.25) (layer B.Cu) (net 16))
 (segment (start 133.985 106.155) (end 135.907 106.155) (width 0.25) (layer F.Cu) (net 16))
 (segment (start 140.462 101.6) (end 135.907 106.155) (width 0.25) (layer F.Cu) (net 16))
 (via (at 140.462 101.6) (size 0.8) (drill 0.4) (layers F.Cu B.Cu) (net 16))
 (segment (start 140.669 101.6) (end 142.367 99.902) (width 0.25) (layer B.Cu) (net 16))
 (segment (start 142.367 99.902) (end 142.16 99.902) (width 0.25) (layer B.Cu) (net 16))
 (segment (start 142.367 100.076) (end 142.367 99.902) (width 0.25) (layer B.Cu) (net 16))
 (segment (start 142.367 99.902) (end 142.367 100.076) (width 0.25) (layer B.Cu) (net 16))
 (segment (start 142.367 99.902) (end 142.367 99.949) (width 0.25) (layer B.Cu) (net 16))
 (segment (start 130.97 102.235) (end 130.97 104.3) (width 0.25) (layer F.Cu) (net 16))
 (segment (start 132.715 106.045) (end 133.875 106.045) (width 0.25) (layer F.Cu) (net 16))
 (segment (start 130.97 104.3) (end 132.715 106.045) (width 0.25) (layer F.Cu) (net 16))
 (segment (start 133.875 106.045) (end 133.985 106.155) (width 0.25) (layer F.Cu) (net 16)))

